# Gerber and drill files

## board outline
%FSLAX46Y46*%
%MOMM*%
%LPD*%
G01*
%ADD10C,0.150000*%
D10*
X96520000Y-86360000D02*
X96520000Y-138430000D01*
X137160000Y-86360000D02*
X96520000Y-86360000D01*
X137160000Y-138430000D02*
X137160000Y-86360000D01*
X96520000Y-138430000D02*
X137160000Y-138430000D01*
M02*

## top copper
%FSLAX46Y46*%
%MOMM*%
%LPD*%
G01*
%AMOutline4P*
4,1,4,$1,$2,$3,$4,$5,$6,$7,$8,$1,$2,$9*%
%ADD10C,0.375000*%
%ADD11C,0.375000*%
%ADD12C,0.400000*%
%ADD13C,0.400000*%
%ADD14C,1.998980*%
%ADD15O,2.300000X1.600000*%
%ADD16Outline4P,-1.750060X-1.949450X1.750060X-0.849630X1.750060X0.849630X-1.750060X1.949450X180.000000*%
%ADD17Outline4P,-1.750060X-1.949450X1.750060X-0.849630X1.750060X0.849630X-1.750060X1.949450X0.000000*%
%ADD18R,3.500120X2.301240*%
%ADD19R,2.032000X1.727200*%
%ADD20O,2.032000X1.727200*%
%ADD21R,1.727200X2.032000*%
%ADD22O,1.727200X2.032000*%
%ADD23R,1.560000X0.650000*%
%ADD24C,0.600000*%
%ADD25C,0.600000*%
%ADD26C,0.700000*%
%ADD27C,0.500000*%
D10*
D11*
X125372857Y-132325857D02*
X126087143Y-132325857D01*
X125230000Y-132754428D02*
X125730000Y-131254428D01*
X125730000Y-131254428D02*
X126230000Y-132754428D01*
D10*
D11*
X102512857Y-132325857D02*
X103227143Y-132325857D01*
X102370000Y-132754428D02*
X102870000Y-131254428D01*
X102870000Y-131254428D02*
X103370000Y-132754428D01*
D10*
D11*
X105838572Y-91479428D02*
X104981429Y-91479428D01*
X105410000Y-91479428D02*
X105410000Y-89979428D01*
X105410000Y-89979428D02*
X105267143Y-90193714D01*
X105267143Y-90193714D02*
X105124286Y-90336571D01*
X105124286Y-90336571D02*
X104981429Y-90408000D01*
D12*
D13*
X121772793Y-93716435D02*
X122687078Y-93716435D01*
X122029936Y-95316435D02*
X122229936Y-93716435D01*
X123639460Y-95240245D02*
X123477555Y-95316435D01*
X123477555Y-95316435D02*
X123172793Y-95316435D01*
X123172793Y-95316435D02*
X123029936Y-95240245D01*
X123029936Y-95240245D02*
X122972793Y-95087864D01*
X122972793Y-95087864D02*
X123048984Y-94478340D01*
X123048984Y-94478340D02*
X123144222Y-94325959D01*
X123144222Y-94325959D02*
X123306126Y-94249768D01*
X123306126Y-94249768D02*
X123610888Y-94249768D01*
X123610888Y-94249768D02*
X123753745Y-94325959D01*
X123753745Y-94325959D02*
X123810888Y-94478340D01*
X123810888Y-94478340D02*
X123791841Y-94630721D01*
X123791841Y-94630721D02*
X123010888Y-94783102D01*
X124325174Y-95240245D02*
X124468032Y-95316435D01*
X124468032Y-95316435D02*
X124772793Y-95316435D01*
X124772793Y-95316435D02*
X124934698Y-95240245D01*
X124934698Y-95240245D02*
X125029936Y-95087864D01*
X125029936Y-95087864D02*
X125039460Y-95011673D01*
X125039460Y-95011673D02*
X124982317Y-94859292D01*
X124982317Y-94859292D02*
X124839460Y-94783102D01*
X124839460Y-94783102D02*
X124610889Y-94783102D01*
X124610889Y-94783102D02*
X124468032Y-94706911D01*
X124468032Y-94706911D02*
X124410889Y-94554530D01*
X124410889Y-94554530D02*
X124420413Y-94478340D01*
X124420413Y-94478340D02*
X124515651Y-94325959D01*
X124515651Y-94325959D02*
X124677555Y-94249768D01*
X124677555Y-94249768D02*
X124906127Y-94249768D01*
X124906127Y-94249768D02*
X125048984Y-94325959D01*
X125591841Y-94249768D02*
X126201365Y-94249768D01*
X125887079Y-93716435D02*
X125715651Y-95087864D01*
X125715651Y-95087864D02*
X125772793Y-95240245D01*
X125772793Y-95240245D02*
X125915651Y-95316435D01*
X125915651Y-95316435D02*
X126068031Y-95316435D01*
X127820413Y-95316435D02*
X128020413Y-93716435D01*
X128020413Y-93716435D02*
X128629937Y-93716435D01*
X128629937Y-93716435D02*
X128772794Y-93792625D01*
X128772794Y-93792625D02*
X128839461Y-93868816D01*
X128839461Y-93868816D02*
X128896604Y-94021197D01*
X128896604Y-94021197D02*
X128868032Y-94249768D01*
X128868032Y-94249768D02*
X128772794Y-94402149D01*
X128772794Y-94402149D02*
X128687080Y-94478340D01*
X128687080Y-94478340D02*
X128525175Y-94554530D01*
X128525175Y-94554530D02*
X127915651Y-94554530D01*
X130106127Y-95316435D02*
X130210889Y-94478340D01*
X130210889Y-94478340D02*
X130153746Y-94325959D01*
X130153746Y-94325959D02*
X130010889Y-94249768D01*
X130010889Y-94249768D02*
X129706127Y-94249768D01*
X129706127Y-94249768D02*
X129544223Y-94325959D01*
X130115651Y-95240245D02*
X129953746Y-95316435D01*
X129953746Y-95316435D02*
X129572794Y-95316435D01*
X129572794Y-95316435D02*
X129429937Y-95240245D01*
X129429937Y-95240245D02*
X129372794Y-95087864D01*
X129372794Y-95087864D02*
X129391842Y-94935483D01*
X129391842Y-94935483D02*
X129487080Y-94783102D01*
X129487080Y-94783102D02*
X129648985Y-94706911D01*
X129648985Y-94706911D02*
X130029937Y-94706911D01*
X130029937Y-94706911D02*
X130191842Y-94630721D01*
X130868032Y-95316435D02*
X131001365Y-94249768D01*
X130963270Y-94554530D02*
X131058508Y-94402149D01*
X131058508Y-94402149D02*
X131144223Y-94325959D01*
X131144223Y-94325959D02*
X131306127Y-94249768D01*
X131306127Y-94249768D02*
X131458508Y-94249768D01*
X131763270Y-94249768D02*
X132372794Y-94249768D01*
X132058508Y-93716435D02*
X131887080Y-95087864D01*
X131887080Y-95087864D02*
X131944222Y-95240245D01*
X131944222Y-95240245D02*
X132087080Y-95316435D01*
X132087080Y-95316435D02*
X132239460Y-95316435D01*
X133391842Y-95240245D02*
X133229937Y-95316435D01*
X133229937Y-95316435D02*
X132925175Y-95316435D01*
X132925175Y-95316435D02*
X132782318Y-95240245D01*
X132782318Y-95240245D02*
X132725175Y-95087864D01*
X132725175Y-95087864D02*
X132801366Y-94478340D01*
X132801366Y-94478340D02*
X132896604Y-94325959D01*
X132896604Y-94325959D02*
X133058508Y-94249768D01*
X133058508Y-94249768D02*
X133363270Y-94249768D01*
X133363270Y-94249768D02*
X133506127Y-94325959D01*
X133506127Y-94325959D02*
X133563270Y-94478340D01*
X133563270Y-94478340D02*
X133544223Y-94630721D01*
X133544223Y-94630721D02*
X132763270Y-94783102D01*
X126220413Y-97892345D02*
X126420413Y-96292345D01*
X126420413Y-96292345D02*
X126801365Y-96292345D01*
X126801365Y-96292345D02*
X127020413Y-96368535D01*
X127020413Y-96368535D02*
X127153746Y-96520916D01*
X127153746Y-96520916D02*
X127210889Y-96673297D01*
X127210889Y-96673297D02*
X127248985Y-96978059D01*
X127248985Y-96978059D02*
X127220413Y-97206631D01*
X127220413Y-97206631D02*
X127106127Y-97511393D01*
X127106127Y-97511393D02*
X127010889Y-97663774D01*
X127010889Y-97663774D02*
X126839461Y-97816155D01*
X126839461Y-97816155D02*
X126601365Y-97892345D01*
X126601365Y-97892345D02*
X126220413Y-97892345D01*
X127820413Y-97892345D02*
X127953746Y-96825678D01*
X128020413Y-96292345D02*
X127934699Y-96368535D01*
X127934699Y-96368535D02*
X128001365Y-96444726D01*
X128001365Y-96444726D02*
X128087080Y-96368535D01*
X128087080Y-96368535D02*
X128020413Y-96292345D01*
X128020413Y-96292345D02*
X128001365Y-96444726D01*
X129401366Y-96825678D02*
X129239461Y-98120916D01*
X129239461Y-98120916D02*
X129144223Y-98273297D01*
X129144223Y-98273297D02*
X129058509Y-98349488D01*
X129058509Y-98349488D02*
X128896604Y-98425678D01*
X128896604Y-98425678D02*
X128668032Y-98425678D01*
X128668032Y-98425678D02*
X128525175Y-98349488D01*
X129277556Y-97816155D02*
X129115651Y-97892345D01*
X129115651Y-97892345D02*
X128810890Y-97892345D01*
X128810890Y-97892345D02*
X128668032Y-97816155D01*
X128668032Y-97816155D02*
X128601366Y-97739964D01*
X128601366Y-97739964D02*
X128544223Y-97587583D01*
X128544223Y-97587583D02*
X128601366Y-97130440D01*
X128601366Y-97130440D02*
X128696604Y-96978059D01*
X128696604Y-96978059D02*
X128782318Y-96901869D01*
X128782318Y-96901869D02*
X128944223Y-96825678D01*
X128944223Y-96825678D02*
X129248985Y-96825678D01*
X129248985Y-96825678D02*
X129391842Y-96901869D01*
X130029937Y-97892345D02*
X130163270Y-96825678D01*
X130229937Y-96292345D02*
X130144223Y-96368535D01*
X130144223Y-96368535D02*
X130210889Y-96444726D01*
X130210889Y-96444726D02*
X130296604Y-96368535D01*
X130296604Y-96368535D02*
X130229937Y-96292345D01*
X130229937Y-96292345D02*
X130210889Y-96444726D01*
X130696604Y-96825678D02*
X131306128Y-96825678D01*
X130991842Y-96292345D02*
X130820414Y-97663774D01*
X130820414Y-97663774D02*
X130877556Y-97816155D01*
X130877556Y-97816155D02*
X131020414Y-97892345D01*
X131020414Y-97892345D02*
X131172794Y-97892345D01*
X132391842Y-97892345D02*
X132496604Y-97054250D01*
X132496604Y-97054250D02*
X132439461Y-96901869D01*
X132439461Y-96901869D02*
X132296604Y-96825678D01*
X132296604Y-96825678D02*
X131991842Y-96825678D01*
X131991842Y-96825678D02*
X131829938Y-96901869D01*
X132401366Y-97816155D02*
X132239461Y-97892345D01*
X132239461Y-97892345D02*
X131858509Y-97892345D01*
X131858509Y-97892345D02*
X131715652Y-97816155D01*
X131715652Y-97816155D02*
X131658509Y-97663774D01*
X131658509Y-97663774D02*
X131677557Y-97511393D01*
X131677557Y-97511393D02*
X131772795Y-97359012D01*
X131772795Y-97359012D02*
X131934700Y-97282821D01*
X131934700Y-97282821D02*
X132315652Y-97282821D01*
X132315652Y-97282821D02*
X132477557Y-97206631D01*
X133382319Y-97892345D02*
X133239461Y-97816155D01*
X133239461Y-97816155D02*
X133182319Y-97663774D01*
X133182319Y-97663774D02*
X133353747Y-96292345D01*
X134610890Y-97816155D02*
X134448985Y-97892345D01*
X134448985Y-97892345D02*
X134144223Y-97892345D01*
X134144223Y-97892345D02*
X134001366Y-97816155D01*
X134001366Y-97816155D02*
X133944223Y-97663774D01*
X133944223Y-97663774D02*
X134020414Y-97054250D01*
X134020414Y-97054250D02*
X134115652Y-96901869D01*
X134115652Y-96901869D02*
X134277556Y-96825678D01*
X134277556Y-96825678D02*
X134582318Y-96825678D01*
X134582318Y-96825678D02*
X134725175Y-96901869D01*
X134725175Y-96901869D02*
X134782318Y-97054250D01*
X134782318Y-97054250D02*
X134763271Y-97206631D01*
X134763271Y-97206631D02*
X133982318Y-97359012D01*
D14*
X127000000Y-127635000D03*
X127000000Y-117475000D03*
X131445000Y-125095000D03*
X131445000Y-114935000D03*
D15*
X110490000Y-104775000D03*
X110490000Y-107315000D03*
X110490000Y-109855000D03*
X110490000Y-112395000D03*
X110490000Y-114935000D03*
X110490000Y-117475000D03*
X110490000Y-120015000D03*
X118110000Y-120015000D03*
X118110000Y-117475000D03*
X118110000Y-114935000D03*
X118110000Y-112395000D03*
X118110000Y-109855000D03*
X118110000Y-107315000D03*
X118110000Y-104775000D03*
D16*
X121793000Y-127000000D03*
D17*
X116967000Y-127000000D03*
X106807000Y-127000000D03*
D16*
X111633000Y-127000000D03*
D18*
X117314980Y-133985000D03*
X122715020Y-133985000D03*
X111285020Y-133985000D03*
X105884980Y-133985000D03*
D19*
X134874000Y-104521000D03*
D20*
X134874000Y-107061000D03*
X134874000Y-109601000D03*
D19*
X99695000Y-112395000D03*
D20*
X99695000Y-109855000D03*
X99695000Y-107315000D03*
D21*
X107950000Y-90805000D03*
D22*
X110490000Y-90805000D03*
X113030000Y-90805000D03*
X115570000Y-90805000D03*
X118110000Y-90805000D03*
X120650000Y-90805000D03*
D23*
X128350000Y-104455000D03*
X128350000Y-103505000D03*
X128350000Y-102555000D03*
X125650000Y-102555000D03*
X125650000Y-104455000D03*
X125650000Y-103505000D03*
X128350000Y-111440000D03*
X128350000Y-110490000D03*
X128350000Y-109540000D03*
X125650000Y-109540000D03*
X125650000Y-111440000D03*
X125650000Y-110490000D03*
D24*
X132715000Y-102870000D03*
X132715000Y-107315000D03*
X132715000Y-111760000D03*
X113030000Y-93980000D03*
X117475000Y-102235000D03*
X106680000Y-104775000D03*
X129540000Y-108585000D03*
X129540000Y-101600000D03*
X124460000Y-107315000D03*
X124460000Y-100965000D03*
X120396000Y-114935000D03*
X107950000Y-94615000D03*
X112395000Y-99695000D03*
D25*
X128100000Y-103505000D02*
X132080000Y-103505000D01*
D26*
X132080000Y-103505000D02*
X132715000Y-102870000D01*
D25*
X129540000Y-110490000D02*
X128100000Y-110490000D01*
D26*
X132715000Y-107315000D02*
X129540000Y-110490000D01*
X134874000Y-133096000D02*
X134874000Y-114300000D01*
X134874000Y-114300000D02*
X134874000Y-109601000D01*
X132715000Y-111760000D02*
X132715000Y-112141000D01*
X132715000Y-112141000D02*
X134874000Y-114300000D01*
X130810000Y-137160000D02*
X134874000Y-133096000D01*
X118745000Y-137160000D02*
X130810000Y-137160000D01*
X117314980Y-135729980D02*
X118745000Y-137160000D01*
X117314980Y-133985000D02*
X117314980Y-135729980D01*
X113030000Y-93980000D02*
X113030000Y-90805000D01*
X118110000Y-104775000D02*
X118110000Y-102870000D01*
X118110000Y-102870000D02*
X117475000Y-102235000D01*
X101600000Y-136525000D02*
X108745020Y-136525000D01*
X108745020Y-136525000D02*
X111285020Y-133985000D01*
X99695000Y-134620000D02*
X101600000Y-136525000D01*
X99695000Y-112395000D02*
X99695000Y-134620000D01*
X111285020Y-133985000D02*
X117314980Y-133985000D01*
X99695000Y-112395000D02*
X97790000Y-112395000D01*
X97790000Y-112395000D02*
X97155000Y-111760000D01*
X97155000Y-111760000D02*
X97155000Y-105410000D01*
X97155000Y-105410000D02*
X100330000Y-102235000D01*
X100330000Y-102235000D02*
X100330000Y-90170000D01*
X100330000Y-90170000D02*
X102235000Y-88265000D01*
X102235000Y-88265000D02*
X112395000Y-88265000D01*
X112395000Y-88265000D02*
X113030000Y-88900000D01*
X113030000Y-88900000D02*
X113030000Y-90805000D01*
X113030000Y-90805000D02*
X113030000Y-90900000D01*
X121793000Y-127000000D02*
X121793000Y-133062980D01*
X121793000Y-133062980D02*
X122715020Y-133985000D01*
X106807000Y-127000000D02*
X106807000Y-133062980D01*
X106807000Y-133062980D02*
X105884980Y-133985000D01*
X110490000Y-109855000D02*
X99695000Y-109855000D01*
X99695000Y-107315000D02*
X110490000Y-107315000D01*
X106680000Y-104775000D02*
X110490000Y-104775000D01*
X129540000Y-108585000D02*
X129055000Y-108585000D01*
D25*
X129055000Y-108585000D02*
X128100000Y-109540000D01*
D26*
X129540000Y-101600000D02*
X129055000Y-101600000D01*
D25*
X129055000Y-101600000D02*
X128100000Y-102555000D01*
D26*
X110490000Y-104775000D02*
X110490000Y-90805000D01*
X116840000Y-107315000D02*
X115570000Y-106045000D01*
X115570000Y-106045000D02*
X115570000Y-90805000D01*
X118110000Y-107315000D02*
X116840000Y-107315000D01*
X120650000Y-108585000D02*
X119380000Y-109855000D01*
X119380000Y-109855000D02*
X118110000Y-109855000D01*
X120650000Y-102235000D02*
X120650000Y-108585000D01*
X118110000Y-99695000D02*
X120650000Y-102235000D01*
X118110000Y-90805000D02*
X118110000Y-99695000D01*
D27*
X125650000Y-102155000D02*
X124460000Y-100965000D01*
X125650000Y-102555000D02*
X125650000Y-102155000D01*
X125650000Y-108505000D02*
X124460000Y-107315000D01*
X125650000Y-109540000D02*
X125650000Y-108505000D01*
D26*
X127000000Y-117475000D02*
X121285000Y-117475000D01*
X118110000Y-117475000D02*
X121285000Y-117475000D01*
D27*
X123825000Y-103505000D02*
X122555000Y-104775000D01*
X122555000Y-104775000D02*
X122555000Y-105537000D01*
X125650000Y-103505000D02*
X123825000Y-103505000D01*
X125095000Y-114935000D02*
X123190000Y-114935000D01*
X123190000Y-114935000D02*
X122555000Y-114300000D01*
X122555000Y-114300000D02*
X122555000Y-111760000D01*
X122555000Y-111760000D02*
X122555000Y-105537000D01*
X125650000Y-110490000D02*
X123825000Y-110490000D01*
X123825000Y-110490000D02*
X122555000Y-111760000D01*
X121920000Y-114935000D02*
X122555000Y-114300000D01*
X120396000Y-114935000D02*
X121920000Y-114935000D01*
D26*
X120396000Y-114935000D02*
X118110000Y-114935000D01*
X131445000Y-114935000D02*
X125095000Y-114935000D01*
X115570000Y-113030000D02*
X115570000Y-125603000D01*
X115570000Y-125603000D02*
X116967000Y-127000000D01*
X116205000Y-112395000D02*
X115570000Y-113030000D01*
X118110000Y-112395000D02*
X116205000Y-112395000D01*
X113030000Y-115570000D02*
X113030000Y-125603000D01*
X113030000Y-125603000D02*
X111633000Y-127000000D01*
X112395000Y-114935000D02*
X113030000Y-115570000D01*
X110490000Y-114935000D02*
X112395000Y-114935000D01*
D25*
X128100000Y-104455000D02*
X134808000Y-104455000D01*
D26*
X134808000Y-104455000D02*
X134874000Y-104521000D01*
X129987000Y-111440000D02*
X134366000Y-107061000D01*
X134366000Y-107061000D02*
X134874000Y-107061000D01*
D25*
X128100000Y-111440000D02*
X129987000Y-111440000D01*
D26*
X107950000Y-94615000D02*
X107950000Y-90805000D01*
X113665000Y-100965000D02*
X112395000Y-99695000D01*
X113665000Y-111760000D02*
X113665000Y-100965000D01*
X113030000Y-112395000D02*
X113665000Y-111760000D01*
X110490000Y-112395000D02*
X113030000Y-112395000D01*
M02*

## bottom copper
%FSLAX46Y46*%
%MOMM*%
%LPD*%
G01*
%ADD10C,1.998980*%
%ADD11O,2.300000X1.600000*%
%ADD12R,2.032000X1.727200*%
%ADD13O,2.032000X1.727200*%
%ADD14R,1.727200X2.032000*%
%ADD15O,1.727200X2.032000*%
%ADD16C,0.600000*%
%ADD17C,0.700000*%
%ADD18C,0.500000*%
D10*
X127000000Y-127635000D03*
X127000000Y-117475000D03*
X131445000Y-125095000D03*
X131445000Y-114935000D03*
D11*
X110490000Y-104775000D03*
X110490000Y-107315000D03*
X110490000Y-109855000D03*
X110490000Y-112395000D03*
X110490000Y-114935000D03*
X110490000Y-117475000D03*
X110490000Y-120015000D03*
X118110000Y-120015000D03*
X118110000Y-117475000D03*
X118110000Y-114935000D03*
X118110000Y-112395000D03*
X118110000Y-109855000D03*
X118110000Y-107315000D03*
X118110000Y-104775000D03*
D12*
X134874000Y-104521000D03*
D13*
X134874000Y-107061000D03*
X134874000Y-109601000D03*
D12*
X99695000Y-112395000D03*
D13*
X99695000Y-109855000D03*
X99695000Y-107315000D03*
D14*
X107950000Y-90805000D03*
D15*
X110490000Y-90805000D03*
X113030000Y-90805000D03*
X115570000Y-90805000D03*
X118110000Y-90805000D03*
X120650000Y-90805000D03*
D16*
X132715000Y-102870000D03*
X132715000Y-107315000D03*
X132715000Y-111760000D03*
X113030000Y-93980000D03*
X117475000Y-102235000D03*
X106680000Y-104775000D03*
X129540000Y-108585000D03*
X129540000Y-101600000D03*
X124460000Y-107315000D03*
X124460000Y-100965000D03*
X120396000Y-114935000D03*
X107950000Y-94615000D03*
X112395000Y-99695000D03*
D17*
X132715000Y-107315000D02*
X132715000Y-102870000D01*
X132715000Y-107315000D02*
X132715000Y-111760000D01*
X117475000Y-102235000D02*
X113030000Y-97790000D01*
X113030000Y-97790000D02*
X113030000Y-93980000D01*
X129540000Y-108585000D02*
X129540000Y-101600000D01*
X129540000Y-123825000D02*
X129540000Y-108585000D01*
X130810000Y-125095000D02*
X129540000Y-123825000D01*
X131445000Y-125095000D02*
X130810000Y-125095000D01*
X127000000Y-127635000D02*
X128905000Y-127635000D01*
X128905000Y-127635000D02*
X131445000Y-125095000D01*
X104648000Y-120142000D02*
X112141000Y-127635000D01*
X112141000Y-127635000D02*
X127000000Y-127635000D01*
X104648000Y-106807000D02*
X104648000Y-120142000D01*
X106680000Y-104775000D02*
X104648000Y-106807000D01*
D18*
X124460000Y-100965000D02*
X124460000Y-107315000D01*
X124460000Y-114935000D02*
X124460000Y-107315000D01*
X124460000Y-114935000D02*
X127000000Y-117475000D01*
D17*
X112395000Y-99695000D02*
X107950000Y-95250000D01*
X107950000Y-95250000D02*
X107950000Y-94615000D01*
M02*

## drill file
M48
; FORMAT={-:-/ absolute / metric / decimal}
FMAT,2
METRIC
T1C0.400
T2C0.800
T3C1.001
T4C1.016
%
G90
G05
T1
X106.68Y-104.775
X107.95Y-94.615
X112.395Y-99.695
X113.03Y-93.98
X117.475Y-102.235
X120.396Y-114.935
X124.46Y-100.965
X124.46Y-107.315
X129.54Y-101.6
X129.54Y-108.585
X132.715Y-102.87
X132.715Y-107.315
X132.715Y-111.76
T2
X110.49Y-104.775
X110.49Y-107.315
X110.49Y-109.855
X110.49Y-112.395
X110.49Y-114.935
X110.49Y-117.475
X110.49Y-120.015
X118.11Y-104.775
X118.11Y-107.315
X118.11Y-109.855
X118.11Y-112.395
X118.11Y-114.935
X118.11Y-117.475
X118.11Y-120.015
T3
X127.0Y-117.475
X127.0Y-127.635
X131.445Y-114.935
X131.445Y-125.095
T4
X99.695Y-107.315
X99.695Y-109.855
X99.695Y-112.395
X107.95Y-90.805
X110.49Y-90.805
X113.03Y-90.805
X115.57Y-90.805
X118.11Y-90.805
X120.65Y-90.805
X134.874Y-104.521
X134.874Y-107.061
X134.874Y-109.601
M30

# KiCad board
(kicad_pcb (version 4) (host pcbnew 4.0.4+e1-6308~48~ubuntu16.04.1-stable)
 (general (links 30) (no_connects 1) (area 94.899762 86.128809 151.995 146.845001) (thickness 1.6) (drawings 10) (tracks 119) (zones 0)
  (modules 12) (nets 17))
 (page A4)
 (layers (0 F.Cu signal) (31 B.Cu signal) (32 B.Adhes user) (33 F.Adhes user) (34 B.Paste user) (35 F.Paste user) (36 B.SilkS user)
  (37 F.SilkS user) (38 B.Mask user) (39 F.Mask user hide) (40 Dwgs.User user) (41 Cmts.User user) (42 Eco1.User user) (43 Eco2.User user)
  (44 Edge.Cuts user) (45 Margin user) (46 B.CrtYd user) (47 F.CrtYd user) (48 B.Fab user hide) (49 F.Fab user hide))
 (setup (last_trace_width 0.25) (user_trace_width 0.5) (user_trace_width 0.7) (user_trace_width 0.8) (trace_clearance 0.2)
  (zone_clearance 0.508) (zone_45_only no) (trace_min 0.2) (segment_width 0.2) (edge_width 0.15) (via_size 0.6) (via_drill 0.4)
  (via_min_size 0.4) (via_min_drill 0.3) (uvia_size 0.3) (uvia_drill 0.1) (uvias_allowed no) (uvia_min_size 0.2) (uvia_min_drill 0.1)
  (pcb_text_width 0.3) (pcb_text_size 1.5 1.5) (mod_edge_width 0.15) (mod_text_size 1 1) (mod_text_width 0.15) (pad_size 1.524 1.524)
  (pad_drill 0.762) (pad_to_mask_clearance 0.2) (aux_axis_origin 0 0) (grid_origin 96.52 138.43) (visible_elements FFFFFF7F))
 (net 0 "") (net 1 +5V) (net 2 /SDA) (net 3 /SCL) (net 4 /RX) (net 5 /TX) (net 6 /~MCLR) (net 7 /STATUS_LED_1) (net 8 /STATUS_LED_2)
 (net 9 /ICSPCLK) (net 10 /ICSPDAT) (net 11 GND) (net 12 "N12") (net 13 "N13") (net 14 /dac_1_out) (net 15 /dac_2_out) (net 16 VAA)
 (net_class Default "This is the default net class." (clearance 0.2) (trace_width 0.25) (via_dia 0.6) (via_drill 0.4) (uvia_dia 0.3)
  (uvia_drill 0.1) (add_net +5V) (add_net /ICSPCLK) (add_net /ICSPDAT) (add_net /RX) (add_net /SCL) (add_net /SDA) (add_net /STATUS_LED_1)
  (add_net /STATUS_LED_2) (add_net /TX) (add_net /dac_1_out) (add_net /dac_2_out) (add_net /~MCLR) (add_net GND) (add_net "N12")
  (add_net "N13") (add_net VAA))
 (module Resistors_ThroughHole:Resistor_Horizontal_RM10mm (layer F.Cu) (at 127 127.635 90)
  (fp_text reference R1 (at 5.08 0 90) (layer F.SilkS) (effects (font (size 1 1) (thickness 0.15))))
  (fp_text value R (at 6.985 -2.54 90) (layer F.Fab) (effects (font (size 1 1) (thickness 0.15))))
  (pad 1 thru_hole circle (at 0 0 90) (size 1.99898 1.99898) (drill 1.00076) (layers *.Cu *.SilkS *.Mask) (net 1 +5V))
  (pad 2 thru_hole circle (at 10.16 0 90) (size 1.99898 1.99898) (drill 1.00076) (layers *.Cu *.SilkS *.Mask) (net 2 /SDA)))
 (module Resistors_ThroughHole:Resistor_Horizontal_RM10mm (layer F.Cu) (at 131.445 125.095 90)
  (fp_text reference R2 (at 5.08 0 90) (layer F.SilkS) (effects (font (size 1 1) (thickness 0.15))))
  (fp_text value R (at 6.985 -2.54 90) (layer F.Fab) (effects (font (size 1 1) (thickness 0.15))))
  (pad 1 thru_hole circle (at 0 0 90) (size 1.99898 1.99898) (drill 1.00076) (layers *.Cu *.SilkS *.Mask) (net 1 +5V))
  (pad 2 thru_hole circle (at 10.16 0 90) (size 1.99898 1.99898) (drill 1.00076) (layers *.Cu *.SilkS *.Mask) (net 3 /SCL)))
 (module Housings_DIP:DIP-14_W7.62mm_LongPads (layer F.Cu) (at 110.49 104.775)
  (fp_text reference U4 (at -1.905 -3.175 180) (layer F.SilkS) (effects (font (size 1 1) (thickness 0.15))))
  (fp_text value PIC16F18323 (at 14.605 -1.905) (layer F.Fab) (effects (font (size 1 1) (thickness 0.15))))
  (pad 1 thru_hole oval (at 0 0) (size 2.3 1.6) (drill 0.8) (layers *.Cu *.Mask F.SilkS) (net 1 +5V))
  (pad 2 thru_hole oval (at 0 2.54) (size 2.3 1.6) (drill 0.8) (layers *.Cu *.Mask F.SilkS) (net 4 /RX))
  (pad 3 thru_hole oval (at 0 5.08) (size 2.3 1.6) (drill 0.8) (layers *.Cu *.Mask F.SilkS) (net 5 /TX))
  (pad 4 thru_hole oval (at 0 7.62) (size 2.3 1.6) (drill 0.8) (layers *.Cu *.Mask F.SilkS) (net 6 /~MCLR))
  (pad 5 thru_hole oval (at 0 10.16) (size 2.3 1.6) (drill 0.8) (layers *.Cu *.Mask F.SilkS) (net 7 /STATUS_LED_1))
  (pad 6 thru_hole oval (at 0 12.7) (size 2.3 1.6) (drill 0.8) (layers *.Cu *.Mask F.SilkS))
  (pad 7 thru_hole oval (at 0 15.24) (size 2.3 1.6) (drill 0.8) (layers *.Cu *.Mask F.SilkS))
  (pad 8 thru_hole oval (at 7.62 15.24) (size 2.3 1.6) (drill 0.8) (layers *.Cu *.Mask F.SilkS))
  (pad 9 thru_hole oval (at 7.62 12.7) (size 2.3 1.6) (drill 0.8) (layers *.Cu *.Mask F.SilkS) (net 2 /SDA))
  (pad 10 thru_hole oval (at 7.62 10.16) (size 2.3 1.6) (drill 0.8) (layers *.Cu *.Mask F.SilkS) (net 3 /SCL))
  (pad 11 thru_hole oval (at 7.62 7.62) (size 2.3 1.6) (drill 0.8) (layers *.Cu *.Mask F.SilkS) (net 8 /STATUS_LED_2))
  (pad 12 thru_hole oval (at 7.62 5.08) (size 2.3 1.6) (drill 0.8) (layers *.Cu *.Mask F.SilkS) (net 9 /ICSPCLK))
  (pad 13 thru_hole oval (at 7.62 2.54) (size 2.3 1.6) (drill 0.8) (layers *.Cu *.Mask F.SilkS) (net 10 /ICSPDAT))
  (pad 14 thru_hole oval (at 7.62 0) (size 2.3 1.6) (drill 0.8) (layers *.Cu *.Mask F.SilkS) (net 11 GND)))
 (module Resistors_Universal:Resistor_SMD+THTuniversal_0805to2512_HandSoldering (layer F.Cu) (at 119.38 127 180)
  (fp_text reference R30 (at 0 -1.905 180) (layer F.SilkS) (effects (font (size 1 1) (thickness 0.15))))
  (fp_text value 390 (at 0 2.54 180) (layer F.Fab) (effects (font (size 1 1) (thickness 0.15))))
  (pad 1 smd trapezoid (at -2.413 0 180) (size 3.50012 2.79908) (rect_delta 1.09982 0) (layers F.Cu F.Paste F.Mask) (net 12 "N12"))
  (pad 2 smd trapezoid (at 2.413 0) (size 3.50012 2.79908) (rect_delta 1.09982 0) (layers F.Cu F.Paste F.Mask) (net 8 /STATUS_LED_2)))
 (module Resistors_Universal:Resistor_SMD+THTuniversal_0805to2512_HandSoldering (layer F.Cu) (at 109.22 127)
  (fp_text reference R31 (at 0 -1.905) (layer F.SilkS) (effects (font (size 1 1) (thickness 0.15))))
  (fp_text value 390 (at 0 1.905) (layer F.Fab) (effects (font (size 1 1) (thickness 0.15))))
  (pad 1 smd trapezoid (at -2.413 0) (size 3.50012 2.79908) (rect_delta 1.09982 0) (layers F.Cu F.Paste F.Mask) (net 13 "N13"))
  (pad 2 smd trapezoid (at 2.413 0 180) (size 3.50012 2.79908) (rect_delta 1.09982 0) (layers F.Cu F.Paste F.Mask) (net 7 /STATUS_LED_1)))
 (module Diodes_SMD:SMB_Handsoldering (layer F.Cu) (at 120.015 133.985)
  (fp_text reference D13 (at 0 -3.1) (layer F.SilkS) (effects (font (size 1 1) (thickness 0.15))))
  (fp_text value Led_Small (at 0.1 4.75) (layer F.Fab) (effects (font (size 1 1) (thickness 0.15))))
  (pad 1 smd rect (at -2.70002 0) (size 3.50012 2.30124) (layers F.Cu F.Paste F.Mask) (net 11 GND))
  (pad 2 smd rect (at 2.70002 0) (size 3.50012 2.30124) (layers F.Cu F.Paste F.Mask) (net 12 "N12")))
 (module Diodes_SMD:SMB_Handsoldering (layer F.Cu) (at 108.585 133.985 180)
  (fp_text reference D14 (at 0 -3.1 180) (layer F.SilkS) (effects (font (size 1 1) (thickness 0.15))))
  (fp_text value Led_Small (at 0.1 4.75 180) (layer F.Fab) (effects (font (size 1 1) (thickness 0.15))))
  (pad 1 smd rect (at -2.70002 0 180) (size 3.50012 2.30124) (layers F.Cu F.Paste F.Mask) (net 11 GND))
  (pad 2 smd rect (at 2.70002 0 180) (size 3.50012 2.30124) (layers F.Cu F.Paste F.Mask) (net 13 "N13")))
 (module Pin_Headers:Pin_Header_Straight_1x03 (layer F.Cu) (at 134.874 104.521)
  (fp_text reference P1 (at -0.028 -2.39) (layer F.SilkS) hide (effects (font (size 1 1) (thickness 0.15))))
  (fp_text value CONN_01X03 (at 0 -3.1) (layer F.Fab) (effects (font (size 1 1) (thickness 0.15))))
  (pad 1 thru_hole rect (at 0 0) (size 2.032 1.7272) (drill 1.016) (layers *.Cu *.Mask F.SilkS) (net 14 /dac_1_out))
  (pad 2 thru_hole oval (at 0 2.54) (size 2.032 1.7272) (drill 1.016) (layers *.Cu *.Mask F.SilkS) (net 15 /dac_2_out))
  (pad 3 thru_hole oval (at 0 5.08) (size 2.032 1.7272) (drill 1.016) (layers *.Cu *.Mask F.SilkS) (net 11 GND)))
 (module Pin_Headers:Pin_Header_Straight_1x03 (layer F.Cu) (at 99.695 112.395 180)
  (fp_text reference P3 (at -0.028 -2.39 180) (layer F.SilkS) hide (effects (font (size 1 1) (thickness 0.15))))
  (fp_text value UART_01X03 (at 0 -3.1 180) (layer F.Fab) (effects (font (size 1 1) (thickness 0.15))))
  (pad 1 thru_hole rect (at 0 0 180) (size 2.032 1.7272) (drill 1.016) (layers *.Cu *.Mask F.SilkS) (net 11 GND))
  (pad 2 thru_hole oval (at 0 2.54 180) (size 2.032 1.7272) (drill 1.016) (layers *.Cu *.Mask F.SilkS) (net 5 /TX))
  (pad 3 thru_hole oval (at 0 5.08 180) (size 2.032 1.7272) (drill 1.016) (layers *.Cu *.Mask F.SilkS) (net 4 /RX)))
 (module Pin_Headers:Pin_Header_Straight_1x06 (layer F.Cu) (at 107.95 90.805 90)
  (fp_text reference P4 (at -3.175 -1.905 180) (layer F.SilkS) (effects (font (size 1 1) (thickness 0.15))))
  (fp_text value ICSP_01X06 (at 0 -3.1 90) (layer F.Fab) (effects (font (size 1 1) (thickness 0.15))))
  (pad 1 thru_hole rect (at 0 0 90) (size 2.032 1.7272) (drill 1.016) (layers *.Cu *.Mask F.SilkS) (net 6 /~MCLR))
  (pad 2 thru_hole oval (at 0 2.54 90) (size 2.032 1.7272) (drill 1.016) (layers *.Cu *.Mask F.SilkS) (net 1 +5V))
  (pad 3 thru_hole oval (at 0 5.08 90) (size 2.032 1.7272) (drill 1.016) (layers *.Cu *.Mask F.SilkS) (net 11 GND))
  (pad 4 thru_hole oval (at 0 7.62 90) (size 2.032 1.7272) (drill 1.016) (layers *.Cu *.Mask F.SilkS) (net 10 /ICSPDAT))
  (pad 5 thru_hole oval (at 0 10.16 90) (size 2.032 1.7272) (drill 1.016) (layers *.Cu *.Mask F.SilkS) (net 9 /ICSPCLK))
  (pad 6 thru_hole oval (at 0 12.7 90) (size 2.032 1.7272) (drill 1.016) (layers *.Cu *.Mask F.SilkS)))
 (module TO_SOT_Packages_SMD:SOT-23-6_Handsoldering (layer F.Cu) (at 127 103.505 180)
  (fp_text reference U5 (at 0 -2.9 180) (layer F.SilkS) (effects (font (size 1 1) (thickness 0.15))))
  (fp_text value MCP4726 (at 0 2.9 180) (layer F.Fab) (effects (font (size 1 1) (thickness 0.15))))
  (pad 1 smd rect (at -1.35 -0.95 180) (size 1.56 0.65) (layers F.Cu F.Paste F.Mask) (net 14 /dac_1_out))
  (pad 2 smd rect (at -1.35 0 180) (size 1.56 0.65) (layers F.Cu F.Paste F.Mask) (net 11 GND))
  (pad 3 smd rect (at -1.35 0.95 180) (size 1.56 0.65) (layers F.Cu F.Paste F.Mask) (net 1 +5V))
  (pad 4 smd rect (at 1.35 0.95 180) (size 1.56 0.65) (layers F.Cu F.Paste F.Mask) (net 2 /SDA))
  (pad 6 smd rect (at 1.35 -0.95 180) (size 1.56 0.65) (layers F.Cu F.Paste F.Mask) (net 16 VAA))
  (pad 5 smd rect (at 1.35 0 180) (size 1.56 0.65) (layers F.Cu F.Paste F.Mask) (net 3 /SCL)))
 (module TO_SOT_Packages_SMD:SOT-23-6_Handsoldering (layer F.Cu) (at 127 110.49 180)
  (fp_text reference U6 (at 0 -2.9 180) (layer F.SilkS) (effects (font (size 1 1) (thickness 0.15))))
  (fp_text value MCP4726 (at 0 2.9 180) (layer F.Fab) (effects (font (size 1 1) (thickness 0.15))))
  (pad 1 smd rect (at -1.35 -0.95 180) (size 1.56 0.65) (layers F.Cu F.Paste F.Mask) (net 15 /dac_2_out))
  (pad 2 smd rect (at -1.35 0 180) (size 1.56 0.65) (layers F.Cu F.Paste F.Mask) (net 11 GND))
  (pad 3 smd rect (at -1.35 0.95 180) (size 1.56 0.65) (layers F.Cu F.Paste F.Mask) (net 1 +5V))
  (pad 4 smd rect (at 1.35 0.95 180) (size 1.56 0.65) (layers F.Cu F.Paste F.Mask) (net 2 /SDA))
  (pad 6 smd rect (at 1.35 -0.95 180) (size 1.56 0.65) (layers F.Cu F.Paste F.Mask) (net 16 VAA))
  (pad 5 smd rect (at 1.35 0 180) (size 1.56 0.65) (layers F.Cu F.Paste F.Mask) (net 3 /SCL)))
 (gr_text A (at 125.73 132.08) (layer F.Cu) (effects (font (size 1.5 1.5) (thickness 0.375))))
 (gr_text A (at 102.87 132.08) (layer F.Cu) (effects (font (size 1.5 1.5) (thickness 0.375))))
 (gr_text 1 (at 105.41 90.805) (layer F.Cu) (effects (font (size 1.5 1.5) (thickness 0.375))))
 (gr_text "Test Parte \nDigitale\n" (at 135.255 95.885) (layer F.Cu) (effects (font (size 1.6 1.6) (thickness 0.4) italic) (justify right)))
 (gr_line (start 96.52 86.36) (end 96.52 138.43) (angle 90) (layer Edge.Cuts) (width 0.15))
 (gr_line (start 137.16 86.36) (end 96.52 86.36) (angle 90) (layer Edge.Cuts) (width 0.15))
 (gr_line (start 137.16 138.43) (end 137.16 86.36) (angle 90) (layer Edge.Cuts) (width 0.15))
 (gr_line (start 96.52 138.43) (end 137.16 138.43) (angle 90) (layer Edge.Cuts) (width 0.15))
 (segment (start 128.1 103.505) (end 132.08 103.505) (width 0.6) (layer F.Cu) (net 11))
 (segment (start 132.08 103.505) (end 132.715 102.87) (width 0.7) (layer F.Cu) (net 11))
 (via (at 132.715 102.87) (size 0.6) (drill 0.4) (layers F.Cu B.Cu) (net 11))
 (segment (start 132.715 107.315) (end 132.715 102.87) (width 0.7) (layer B.Cu) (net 11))
 (via (at 132.715 107.315) (size 0.6) (drill 0.4) (layers F.Cu B.Cu) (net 11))
 (segment (start 129.54 110.49) (end 128.1 110.49) (width 0.6) (layer F.Cu) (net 11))
 (segment (start 132.715 107.315) (end 129.54 110.49) (width 0.7) (layer F.Cu) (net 11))
 (segment (start 132.715 107.315) (end 132.715 111.76) (width 0.7) (layer B.Cu) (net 11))
 (segment (start 134.874 133.096) (end 134.874 114.3) (width 0.7) (layer F.Cu) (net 11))
 (segment (start 134.874 114.3) (end 134.874 109.601) (width 0.7) (layer F.Cu) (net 11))
 (segment (start 132.715 111.76) (end 132.715 112.141) (width 0.7) (layer F.Cu) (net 11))
 (segment (start 132.715 112.141) (end 134.874 114.3) (width 0.7) (layer F.Cu) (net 11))
 (via (at 132.715 111.76) (size 0.6) (drill 0.4) (layers F.Cu B.Cu) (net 11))
 (segment (start 130.81 137.16) (end 134.874 133.096) (width 0.7) (layer F.Cu) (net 11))
 (segment (start 118.745 137.16) (end 130.81 137.16) (width 0.7) (layer F.Cu) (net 11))
 (segment (start 117.31498 135.72998) (end 118.745 137.16) (width 0.7) (layer F.Cu) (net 11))
 (segment (start 117.31498 133.985) (end 117.31498 135.72998) (width 0.7) (layer F.Cu) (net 11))
 (segment (start 113.03 93.98) (end 113.03 90.805) (width 0.7) (layer F.Cu) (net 11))
 (segment (start 117.475 102.235) (end 113.03 97.79) (width 0.7) (layer B.Cu) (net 11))
 (segment (start 113.03 97.79) (end 113.03 93.98) (width 0.7) (layer B.Cu) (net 11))
 (via (at 113.03 93.98) (size 0.6) (drill 0.4) (layers F.Cu B.Cu) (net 11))
 (segment (start 118.11 104.775) (end 118.11 102.87) (width 0.7) (layer F.Cu) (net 11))
 (segment (start 118.11 102.87) (end 117.475 102.235) (width 0.7) (layer F.Cu) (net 11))
 (via (at 117.475 102.235) (size 0.6) (drill 0.4) (layers F.Cu B.Cu) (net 11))
 (segment (start 101.6 136.525) (end 108.74502 136.525) (width 0.7) (layer F.Cu) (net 11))
 (segment (start 108.74502 136.525) (end 111.28502 133.985) (width 0.7) (layer F.Cu) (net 11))
 (segment (start 99.695 134.62) (end 101.6 136.525) (width 0.7) (layer F.Cu) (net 11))
 (segment (start 99.695 112.395) (end 99.695 134.62) (width 0.7) (layer F.Cu) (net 11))
 (segment (start 111.28502 133.985) (end 117.31498 133.985) (width 0.7) (layer F.Cu) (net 11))
 (segment (start 99.695 112.395) (end 97.79 112.395) (width 0.7) (layer F.Cu) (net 11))
 (segment (start 97.79 112.395) (end 97.155 111.76) (width 0.7) (layer F.Cu) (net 11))
 (segment (start 97.155 111.76) (end 97.155 105.41) (width 0.7) (layer F.Cu) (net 11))
 (segment (start 97.155 105.41) (end 100.33 102.235) (width 0.7) (layer F.Cu) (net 11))
 (segment (start 100.33 102.235) (end 100.33 90.17) (width 0.7) (layer F.Cu) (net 11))
 (segment (start 100.33 90.17) (end 102.235 88.265) (width 0.7) (layer F.Cu) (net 11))
 (segment (start 102.235 88.265) (end 112.395 88.265) (width 0.7) (layer F.Cu) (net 11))
 (segment (start 112.395 88.265) (end 113.03 88.9) (width 0.7) (layer F.Cu) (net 11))
 (segment (start 113.03 88.9) (end 113.03 90.805) (width 0.7) (layer F.Cu) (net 11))
 (segment (start 113.03 90.805) (end 113.03 90.9) (width 0.7) (layer F.Cu) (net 11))
 (segment (start 121.793 127) (end 121.793 133.06298) (width 0.7) (layer F.Cu) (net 12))
 (segment (start 121.793 133.06298) (end 122.71502 133.985) (width 0.7) (layer F.Cu) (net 12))
 (segment (start 106.807 127) (end 106.807 133.06298) (width 0.7) (layer F.Cu) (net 13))
 (segment (start 106.807 133.06298) (end 105.88498 133.985) (width 0.7) (layer F.Cu) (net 13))
 (segment (start 110.49 109.855) (end 99.695 109.855) (width 0.7) (layer F.Cu) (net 5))
 (segment (start 99.695 107.315) (end 110.49 107.315) (width 0.7) (layer F.Cu) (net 4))
 (segment (start 106.68 104.775) (end 110.49 104.775) (width 0.7) (layer F.Cu) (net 1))
 (via (at 106.68 104.775) (size 0.6) (drill 0.4) (layers F.Cu B.Cu) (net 1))
 (segment (start 129.54 108.585) (end 129.055 108.585) (width 0.7) (layer F.Cu) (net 1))
 (segment (start 129.055 108.585) (end 128.1 109.54) (width 0.6) (layer F.Cu) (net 1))
 (segment (start 129.54 108.585) (end 129.54 101.6) (width 0.7) (layer B.Cu) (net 1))
 (segment (start 129.54 123.825) (end 129.54 108.585) (width 0.7) (layer B.Cu) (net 1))
 (via (at 129.54 108.585) (size 0.6) (drill 0.4) (layers F.Cu B.Cu) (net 1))
 (segment (start 129.54 101.6) (end 129.055 101.6) (width 0.7) (layer F.Cu) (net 1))
 (segment (start 129.055 101.6) (end 128.1 102.555) (width 0.6) (layer F.Cu) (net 1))
 (via (at 129.54 101.6) (size 0.6) (drill 0.4) (layers F.Cu B.Cu) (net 1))
 (segment (start 130.81 125.095) (end 129.54 123.825) (width 0.7) (layer B.Cu) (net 1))
 (segment (start 131.445 125.095) (end 130.81 125.095) (width 0.7) (layer B.Cu) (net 1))
 (segment (start 127 127.635) (end 128.905 127.635) (width 0.7) (layer B.Cu) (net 1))
 (segment (start 128.905 127.635) (end 131.445 125.095) (width 0.7) (layer B.Cu) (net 1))
 (segment (start 104.648 120.142) (end 112.141 127.635) (width 0.7) (layer B.Cu) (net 1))
 (segment (start 112.141 127.635) (end 127 127.635) (width 0.7) (layer B.Cu) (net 1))
 (segment (start 104.648 106.807) (end 104.648 120.142) (width 0.7) (layer B.Cu) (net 1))
 (segment (start 106.68 104.775) (end 104.648 106.807) (width 0.7) (layer B.Cu) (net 1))
 (segment (start 110.49 104.775) (end 110.49 90.805) (width 0.7) (layer F.Cu) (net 1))
 (segment (start 116.84 107.315) (end 115.57 106.045) (width 0.7) (layer F.Cu) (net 10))
 (segment (start 115.57 106.045) (end 115.57 90.805) (width 0.7) (layer F.Cu) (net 10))
 (segment (start 118.11 107.315) (end 116.84 107.315) (width 0.7) (layer F.Cu) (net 10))
 (segment (start 120.65 108.585) (end 119.38 109.855) (width 0.7) (layer F.Cu) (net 9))
 (segment (start 119.38 109.855) (end 118.11 109.855) (width 0.7) (layer F.Cu) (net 9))
 (segment (start 120.65 102.235) (end 120.65 108.585) (width 0.7) (layer F.Cu) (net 9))
 (segment (start 118.11 99.695) (end 120.65 102.235) (width 0.7) (layer F.Cu) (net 9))
 (segment (start 118.11 90.805) (end 118.11 99.695) (width 0.7) (layer F.Cu) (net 9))
 (segment (start 124.46 100.965) (end 124.46 107.315) (width 0.5) (layer B.Cu) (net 2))
 (segment (start 124.46 114.935) (end 124.46 107.315) (width 0.5) (layer B.Cu) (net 2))
 (via (at 124.46 107.315) (size 0.6) (drill 0.4) (layers F.Cu B.Cu) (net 2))
 (segment (start 124.46 114.935) (end 127 117.475) (width 0.5) (layer B.Cu) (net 2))
 (via (at 124.46 100.965) (size 0.6) (drill 0.4) (layers F.Cu B.Cu) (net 2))
 (segment (start 125.65 102.155) (end 124.46 100.965) (width 0.5) (layer F.Cu) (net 2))
 (segment (start 125.65 102.555) (end 125.65 102.155) (width 0.5) (layer F.Cu) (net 2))
 (segment (start 125.65 108.505) (end 124.46 107.315) (width 0.5) (layer F.Cu) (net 2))
 (segment (start 125.65 109.54) (end 125.65 108.505) (width 0.5) (layer F.Cu) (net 2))
 (segment (start 127 117.475) (end 121.285 117.475) (width 0.7) (layer F.Cu) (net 2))
 (segment (start 118.11 117.475) (end 121.285 117.475) (width 0.7) (layer F.Cu) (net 2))
 (segment (start 123.825 103.505) (end 122.555 104.775) (width 0.5) (layer F.Cu) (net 3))
 (segment (start 122.555 104.775) (end 122.555 105.537) (width 0.5) (layer F.Cu) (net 3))
 (segment (start 125.65 103.505) (end 123.825 103.505) (width 0.5) (layer F.Cu) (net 3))
 (segment (start 125.095 114.935) (end 123.19 114.935) (width 0.5) (layer F.Cu) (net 3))
 (segment (start 123.19 114.935) (end 122.555 114.3) (width 0.5) (layer F.Cu) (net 3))
 (segment (start 122.555 114.3) (end 122.555 111.76) (width 0.5) (layer F.Cu) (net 3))
 (segment (start 122.555 111.76) (end 122.555 105.537) (width 0.5) (layer F.Cu) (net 3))
 (segment (start 125.65 110.49) (end 123.825 110.49) (width 0.5) (layer F.Cu) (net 3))
 (segment (start 123.825 110.49) (end 122.555 111.76) (width 0.5) (layer F.Cu) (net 3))
 (segment (start 121.92 114.935) (end 122.555 114.3) (width 0.5) (layer F.Cu) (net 3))
 (segment (start 120.396 114.935) (end 121.92 114.935) (width 0.5) (layer F.Cu) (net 3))
 (segment (start 120.396 114.935) (end 118.11 114.935) (width 0.7) (layer F.Cu) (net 3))
 (via (at 120.396 114.935) (size 0.6) (drill 0.4) (layers F.Cu B.Cu) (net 3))
 (segment (start 131.445 114.935) (end 125.095 114.935) (width 0.7) (layer F.Cu) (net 3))
 (segment (start 115.57 113.03) (end 115.57 125.603) (width 0.7) (layer F.Cu) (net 8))
 (segment (start 115.57 125.603) (end 116.967 127) (width 0.7) (layer F.Cu) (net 8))
 (segment (start 116.205 112.395) (end 115.57 113.03) (width 0.7) (layer F.Cu) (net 8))
 (segment (start 118.11 112.395) (end 116.205 112.395) (width 0.7) (layer F.Cu) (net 8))
 (segment (start 113.03 115.57) (end 113.03 125.603) (width 0.7) (layer F.Cu) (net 7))
 (segment (start 113.03 125.603) (end 111.633 127) (width 0.7) (layer F.Cu) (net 7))
 (segment (start 112.395 114.935) (end 113.03 115.57) (width 0.7) (layer F.Cu) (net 7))
 (segment (start 110.49 114.935) (end 112.395 114.935) (width 0.7) (layer F.Cu) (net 7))
 (segment (start 128.1 104.455) (end 134.808 104.455) (width 0.6) (layer F.Cu) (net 14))
 (segment (start 134.808 104.455) (end 134.874 104.521) (width 0.7) (layer F.Cu) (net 14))
 (segment (start 129.987 111.44) (end 134.366 107.061) (width 0.7) (layer F.Cu) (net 15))
 (segment (start 134.366 107.061) (end 134.874 107.061) (width 0.7) (layer F.Cu) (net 15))
 (segment (start 128.1 111.44) (end 129.987 111.44) (width 0.6) (layer F.Cu) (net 15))
 (segment (start 107.95 94.615) (end 107.95 90.805) (width 0.7) (layer F.Cu) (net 6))
 (segment (start 112.395 99.695) (end 107.95 95.25) (width 0.7) (layer B.Cu) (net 6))
 (segment (start 107.95 95.25) (end 107.95 94.615) (width 0.7) (layer B.Cu) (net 6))
 (via (at 107.95 94.615) (size 0.6) (drill 0.4) (layers F.Cu B.Cu) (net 6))
 (segment (start 113.665 100.965) (end 112.395 99.695) (width 0.7) (layer F.Cu) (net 6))
 (via (at 112.395 99.695) (size 0.6) (drill 0.4) (layers F.Cu B.Cu) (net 6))
 (segment (start 113.665 111.76) (end 113.665 100.965) (width 0.7) (layer F.Cu) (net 6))
 (segment (start 113.03 112.395) (end 113.665 111.76) (width 0.7) (layer F.Cu) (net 6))
 (segment (start 110.49 112.395) (end 113.03 112.395) (width 0.7) (layer F.Cu) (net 6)))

